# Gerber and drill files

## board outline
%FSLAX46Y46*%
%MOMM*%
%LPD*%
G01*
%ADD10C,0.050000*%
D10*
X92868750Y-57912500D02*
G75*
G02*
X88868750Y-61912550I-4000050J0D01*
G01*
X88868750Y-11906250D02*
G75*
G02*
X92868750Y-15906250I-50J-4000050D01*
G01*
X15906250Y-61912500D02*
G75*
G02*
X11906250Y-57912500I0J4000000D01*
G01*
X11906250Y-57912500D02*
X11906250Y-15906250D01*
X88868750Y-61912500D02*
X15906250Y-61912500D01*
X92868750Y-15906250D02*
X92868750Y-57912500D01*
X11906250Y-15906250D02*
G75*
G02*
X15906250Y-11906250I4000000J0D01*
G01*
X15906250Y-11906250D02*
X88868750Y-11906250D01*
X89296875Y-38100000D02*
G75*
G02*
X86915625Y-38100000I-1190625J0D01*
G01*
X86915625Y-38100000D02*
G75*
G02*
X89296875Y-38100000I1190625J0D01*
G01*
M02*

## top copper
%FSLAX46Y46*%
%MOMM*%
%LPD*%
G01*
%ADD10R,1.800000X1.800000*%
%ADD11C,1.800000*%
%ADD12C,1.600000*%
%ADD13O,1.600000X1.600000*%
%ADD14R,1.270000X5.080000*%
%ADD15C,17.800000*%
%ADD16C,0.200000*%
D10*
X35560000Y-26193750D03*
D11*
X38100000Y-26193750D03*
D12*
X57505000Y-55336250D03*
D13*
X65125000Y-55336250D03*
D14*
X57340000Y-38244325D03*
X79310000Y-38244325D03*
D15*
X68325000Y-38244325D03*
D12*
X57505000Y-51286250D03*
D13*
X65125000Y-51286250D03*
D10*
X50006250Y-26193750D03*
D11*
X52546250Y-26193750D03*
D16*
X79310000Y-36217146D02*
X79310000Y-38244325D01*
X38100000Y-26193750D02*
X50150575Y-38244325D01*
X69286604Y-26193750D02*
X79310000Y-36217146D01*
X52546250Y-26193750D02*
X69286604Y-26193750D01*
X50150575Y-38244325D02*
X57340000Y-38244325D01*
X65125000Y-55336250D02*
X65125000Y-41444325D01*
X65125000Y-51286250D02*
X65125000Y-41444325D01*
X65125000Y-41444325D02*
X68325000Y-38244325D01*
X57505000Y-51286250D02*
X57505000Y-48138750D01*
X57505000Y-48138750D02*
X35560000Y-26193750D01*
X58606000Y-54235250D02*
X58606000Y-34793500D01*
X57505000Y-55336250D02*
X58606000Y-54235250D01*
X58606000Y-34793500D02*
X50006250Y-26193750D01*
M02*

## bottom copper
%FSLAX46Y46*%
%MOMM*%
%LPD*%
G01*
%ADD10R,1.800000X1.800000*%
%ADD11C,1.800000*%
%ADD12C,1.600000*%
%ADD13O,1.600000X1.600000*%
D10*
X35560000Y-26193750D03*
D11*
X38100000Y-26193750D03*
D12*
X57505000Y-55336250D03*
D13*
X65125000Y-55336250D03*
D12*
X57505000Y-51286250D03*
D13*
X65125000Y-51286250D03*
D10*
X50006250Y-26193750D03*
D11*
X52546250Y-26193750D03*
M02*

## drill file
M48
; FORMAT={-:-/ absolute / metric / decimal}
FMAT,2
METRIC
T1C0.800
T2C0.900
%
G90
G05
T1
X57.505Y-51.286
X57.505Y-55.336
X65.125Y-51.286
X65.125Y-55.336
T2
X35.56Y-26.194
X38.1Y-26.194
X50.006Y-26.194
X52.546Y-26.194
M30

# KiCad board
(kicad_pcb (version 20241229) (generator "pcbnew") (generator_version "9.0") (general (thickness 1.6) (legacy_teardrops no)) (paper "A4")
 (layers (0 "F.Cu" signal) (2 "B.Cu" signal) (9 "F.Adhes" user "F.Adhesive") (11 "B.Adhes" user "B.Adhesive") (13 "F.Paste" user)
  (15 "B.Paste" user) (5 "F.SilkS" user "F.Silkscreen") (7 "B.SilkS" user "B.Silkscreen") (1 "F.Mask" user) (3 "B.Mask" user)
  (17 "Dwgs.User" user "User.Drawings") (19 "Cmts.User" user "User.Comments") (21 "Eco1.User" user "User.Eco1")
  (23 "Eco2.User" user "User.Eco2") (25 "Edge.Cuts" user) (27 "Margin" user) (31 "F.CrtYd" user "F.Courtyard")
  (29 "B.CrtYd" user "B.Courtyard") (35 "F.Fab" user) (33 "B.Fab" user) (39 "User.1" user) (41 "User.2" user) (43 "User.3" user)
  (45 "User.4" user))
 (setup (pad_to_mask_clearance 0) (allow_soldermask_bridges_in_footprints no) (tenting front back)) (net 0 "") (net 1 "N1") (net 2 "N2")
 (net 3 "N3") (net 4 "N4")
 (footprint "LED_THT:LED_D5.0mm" (layer "F.Cu") (at 35.56 26.19375)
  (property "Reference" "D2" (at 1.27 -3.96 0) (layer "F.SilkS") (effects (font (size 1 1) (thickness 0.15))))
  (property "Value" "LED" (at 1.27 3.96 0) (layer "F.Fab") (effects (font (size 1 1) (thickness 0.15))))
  (pad "1" thru_hole rect (at 0 0) (size 1.8 1.8) (drill 0.9) (layers "*.Cu" "*.Mask") (remove_unused_layers no) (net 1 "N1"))
  (pad "2" thru_hole circle (at 2.54 0) (size 1.8 1.8) (drill 0.9) (layers "*.Cu" "*.Mask") (remove_unused_layers no) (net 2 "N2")))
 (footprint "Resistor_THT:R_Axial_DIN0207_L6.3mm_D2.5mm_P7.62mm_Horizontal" (layer "F.Cu") (at 57.505 55.33625)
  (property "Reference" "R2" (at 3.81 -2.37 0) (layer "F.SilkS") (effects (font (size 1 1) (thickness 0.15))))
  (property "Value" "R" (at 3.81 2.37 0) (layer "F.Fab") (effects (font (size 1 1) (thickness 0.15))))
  (pad "1" thru_hole circle (at 0 0) (size 1.6 1.6) (drill 0.8) (layers "*.Cu" "*.Mask") (remove_unused_layers no) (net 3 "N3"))
  (pad "2" thru_hole oval (at 7.62 0) (size 1.6 1.6) (drill 0.8) (layers "*.Cu" "*.Mask") (remove_unused_layers no) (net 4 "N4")))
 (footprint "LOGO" (layer "F.Cu") (at 38.1 50.00625)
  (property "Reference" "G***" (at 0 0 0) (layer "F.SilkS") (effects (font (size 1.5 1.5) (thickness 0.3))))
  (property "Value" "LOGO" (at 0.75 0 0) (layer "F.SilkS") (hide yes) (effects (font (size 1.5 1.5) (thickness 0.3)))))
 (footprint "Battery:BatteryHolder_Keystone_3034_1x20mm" (layer "F.Cu") (at 68.325 38.244325)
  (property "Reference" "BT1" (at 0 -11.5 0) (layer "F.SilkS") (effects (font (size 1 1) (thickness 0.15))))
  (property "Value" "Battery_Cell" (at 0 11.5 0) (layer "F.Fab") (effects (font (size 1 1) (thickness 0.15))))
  (pad "1" smd rect (at -10.985 0) (size 1.27 5.08) (layers "F.Cu" "F.Mask" "F.Paste") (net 2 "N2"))
  (pad "1" smd rect (at 10.985 0) (size 1.27 5.08) (layers "F.Cu" "F.Mask" "F.Paste") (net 2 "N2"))
  (pad "2" smd circle (at 0 0) (size 17.8 17.8) (layers "F.Cu" "F.Mask") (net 4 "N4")))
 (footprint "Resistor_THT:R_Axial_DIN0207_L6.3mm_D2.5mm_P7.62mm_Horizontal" (layer "F.Cu") (at 57.505 51.28625)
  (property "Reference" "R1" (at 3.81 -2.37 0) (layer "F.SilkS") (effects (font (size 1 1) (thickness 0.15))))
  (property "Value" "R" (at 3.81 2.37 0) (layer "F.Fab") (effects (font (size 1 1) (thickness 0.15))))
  (pad "1" thru_hole circle (at 0 0) (size 1.6 1.6) (drill 0.8) (layers "*.Cu" "*.Mask") (remove_unused_layers no) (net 1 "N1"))
  (pad "2" thru_hole oval (at 7.62 0) (size 1.6 1.6) (drill 0.8) (layers "*.Cu" "*.Mask") (remove_unused_layers no) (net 4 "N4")))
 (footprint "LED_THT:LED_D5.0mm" (layer "F.Cu") (at 50.00625 26.19375)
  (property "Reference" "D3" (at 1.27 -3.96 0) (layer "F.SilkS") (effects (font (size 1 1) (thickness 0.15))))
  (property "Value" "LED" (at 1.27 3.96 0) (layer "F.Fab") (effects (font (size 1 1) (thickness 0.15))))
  (pad "1" thru_hole rect (at 0 0) (size 1.8 1.8) (drill 0.9) (layers "*.Cu" "*.Mask") (remove_unused_layers no) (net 3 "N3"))
  (pad "2" thru_hole circle (at 2.54 0) (size 1.8 1.8) (drill 0.9) (layers "*.Cu" "*.Mask") (remove_unused_layers no) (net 2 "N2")))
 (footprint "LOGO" (layer "B.Cu") (at 26.19375 19.05 180)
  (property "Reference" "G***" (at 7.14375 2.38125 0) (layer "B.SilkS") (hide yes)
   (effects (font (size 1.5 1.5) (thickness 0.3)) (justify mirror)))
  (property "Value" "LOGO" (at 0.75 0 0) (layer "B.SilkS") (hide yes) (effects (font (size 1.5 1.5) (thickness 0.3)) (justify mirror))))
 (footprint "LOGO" (layer "B.Cu") (at 21.43125 40.48125 180)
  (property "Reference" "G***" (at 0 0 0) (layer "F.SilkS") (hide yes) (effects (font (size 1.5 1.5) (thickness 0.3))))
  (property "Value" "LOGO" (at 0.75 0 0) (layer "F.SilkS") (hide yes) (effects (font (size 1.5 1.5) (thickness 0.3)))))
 (gr_arc (start 92.86875 57.9125) (mid 91.697177 60.740927) (end 88.86875 61.9125) (stroke (width 0.05) (type default)) (layer "Edge.Cuts"))
 (gr_arc (start 88.86875 11.90625) (mid 91.697177 13.077823) (end 92.86875 15.90625) (stroke (width 0.05) (type default))
  (layer "Edge.Cuts"))
 (gr_arc (start 15.90625 61.9125) (mid 13.077823 60.740927) (end 11.90625 57.9125) (stroke (width 0.05) (type default)) (layer "Edge.Cuts"))
 (gr_line (start 11.90625 57.9125) (end 11.90625 15.90625) (stroke (width 0.05) (type default)) (layer "Edge.Cuts"))
 (gr_line (start 88.86875 61.9125) (end 15.90625 61.9125) (stroke (width 0.05) (type default)) (layer "Edge.Cuts"))
 (gr_line (start 92.86875 15.90625) (end 92.86875 57.9125) (stroke (width 0.05) (type default)) (layer "Edge.Cuts"))
 (gr_arc (start 11.90625 15.90625) (mid 13.077823 13.077823) (end 15.90625 11.90625) (stroke (width 0.05) (type default))
  (layer "Edge.Cuts"))
 (gr_line (start 15.90625 11.90625) (end 88.86875 11.90625) (stroke (width 0.05) (type default)) (layer "Edge.Cuts"))
 (gr_circle (center 88.10625 38.1) (end 88.10625 39.290625) (stroke (width 0.05) (type default)) (fill no) (layer "Edge.Cuts"))
 (segment (start 79.31 36.217146) (end 79.31 38.244325) (width 0.2) (layer "F.Cu") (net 2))
 (segment (start 38.1 26.19375) (end 50.150575 38.244325) (width 0.2) (layer "F.Cu") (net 2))
 (segment (start 69.286604 26.19375) (end 79.31 36.217146) (width 0.2) (layer "F.Cu") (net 2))
 (segment (start 52.54625 26.19375) (end 69.286604 26.19375) (width 0.2) (layer "F.Cu") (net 2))
 (segment (start 50.150575 38.244325) (end 57.34 38.244325) (width 0.2) (layer "F.Cu") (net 2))
 (segment (start 65.125 55.33625) (end 65.125 41.444325) (width 0.2) (layer "F.Cu") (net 4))
 (segment (start 65.125 51.28625) (end 65.125 41.444325) (width 0.2) (layer "F.Cu") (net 4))
 (segment (start 65.125 41.444325) (end 68.325 38.244325) (width 0.2) (layer "F.Cu") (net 4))
 (segment (start 57.505 51.28625) (end 57.505 48.13875) (width 0.2) (layer "F.Cu") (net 1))
 (segment (start 57.505 48.13875) (end 35.56 26.19375) (width 0.2) (layer "F.Cu") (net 1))
 (segment (start 58.606 54.23525) (end 58.606 34.7935) (width 0.2) (layer "F.Cu") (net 3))
 (segment (start 57.505 55.33625) (end 58.606 54.23525) (width 0.2) (layer "F.Cu") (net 3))
 (segment (start 58.606 34.7935) (end 50.00625 26.19375) (width 0.2) (layer "F.Cu") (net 3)))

